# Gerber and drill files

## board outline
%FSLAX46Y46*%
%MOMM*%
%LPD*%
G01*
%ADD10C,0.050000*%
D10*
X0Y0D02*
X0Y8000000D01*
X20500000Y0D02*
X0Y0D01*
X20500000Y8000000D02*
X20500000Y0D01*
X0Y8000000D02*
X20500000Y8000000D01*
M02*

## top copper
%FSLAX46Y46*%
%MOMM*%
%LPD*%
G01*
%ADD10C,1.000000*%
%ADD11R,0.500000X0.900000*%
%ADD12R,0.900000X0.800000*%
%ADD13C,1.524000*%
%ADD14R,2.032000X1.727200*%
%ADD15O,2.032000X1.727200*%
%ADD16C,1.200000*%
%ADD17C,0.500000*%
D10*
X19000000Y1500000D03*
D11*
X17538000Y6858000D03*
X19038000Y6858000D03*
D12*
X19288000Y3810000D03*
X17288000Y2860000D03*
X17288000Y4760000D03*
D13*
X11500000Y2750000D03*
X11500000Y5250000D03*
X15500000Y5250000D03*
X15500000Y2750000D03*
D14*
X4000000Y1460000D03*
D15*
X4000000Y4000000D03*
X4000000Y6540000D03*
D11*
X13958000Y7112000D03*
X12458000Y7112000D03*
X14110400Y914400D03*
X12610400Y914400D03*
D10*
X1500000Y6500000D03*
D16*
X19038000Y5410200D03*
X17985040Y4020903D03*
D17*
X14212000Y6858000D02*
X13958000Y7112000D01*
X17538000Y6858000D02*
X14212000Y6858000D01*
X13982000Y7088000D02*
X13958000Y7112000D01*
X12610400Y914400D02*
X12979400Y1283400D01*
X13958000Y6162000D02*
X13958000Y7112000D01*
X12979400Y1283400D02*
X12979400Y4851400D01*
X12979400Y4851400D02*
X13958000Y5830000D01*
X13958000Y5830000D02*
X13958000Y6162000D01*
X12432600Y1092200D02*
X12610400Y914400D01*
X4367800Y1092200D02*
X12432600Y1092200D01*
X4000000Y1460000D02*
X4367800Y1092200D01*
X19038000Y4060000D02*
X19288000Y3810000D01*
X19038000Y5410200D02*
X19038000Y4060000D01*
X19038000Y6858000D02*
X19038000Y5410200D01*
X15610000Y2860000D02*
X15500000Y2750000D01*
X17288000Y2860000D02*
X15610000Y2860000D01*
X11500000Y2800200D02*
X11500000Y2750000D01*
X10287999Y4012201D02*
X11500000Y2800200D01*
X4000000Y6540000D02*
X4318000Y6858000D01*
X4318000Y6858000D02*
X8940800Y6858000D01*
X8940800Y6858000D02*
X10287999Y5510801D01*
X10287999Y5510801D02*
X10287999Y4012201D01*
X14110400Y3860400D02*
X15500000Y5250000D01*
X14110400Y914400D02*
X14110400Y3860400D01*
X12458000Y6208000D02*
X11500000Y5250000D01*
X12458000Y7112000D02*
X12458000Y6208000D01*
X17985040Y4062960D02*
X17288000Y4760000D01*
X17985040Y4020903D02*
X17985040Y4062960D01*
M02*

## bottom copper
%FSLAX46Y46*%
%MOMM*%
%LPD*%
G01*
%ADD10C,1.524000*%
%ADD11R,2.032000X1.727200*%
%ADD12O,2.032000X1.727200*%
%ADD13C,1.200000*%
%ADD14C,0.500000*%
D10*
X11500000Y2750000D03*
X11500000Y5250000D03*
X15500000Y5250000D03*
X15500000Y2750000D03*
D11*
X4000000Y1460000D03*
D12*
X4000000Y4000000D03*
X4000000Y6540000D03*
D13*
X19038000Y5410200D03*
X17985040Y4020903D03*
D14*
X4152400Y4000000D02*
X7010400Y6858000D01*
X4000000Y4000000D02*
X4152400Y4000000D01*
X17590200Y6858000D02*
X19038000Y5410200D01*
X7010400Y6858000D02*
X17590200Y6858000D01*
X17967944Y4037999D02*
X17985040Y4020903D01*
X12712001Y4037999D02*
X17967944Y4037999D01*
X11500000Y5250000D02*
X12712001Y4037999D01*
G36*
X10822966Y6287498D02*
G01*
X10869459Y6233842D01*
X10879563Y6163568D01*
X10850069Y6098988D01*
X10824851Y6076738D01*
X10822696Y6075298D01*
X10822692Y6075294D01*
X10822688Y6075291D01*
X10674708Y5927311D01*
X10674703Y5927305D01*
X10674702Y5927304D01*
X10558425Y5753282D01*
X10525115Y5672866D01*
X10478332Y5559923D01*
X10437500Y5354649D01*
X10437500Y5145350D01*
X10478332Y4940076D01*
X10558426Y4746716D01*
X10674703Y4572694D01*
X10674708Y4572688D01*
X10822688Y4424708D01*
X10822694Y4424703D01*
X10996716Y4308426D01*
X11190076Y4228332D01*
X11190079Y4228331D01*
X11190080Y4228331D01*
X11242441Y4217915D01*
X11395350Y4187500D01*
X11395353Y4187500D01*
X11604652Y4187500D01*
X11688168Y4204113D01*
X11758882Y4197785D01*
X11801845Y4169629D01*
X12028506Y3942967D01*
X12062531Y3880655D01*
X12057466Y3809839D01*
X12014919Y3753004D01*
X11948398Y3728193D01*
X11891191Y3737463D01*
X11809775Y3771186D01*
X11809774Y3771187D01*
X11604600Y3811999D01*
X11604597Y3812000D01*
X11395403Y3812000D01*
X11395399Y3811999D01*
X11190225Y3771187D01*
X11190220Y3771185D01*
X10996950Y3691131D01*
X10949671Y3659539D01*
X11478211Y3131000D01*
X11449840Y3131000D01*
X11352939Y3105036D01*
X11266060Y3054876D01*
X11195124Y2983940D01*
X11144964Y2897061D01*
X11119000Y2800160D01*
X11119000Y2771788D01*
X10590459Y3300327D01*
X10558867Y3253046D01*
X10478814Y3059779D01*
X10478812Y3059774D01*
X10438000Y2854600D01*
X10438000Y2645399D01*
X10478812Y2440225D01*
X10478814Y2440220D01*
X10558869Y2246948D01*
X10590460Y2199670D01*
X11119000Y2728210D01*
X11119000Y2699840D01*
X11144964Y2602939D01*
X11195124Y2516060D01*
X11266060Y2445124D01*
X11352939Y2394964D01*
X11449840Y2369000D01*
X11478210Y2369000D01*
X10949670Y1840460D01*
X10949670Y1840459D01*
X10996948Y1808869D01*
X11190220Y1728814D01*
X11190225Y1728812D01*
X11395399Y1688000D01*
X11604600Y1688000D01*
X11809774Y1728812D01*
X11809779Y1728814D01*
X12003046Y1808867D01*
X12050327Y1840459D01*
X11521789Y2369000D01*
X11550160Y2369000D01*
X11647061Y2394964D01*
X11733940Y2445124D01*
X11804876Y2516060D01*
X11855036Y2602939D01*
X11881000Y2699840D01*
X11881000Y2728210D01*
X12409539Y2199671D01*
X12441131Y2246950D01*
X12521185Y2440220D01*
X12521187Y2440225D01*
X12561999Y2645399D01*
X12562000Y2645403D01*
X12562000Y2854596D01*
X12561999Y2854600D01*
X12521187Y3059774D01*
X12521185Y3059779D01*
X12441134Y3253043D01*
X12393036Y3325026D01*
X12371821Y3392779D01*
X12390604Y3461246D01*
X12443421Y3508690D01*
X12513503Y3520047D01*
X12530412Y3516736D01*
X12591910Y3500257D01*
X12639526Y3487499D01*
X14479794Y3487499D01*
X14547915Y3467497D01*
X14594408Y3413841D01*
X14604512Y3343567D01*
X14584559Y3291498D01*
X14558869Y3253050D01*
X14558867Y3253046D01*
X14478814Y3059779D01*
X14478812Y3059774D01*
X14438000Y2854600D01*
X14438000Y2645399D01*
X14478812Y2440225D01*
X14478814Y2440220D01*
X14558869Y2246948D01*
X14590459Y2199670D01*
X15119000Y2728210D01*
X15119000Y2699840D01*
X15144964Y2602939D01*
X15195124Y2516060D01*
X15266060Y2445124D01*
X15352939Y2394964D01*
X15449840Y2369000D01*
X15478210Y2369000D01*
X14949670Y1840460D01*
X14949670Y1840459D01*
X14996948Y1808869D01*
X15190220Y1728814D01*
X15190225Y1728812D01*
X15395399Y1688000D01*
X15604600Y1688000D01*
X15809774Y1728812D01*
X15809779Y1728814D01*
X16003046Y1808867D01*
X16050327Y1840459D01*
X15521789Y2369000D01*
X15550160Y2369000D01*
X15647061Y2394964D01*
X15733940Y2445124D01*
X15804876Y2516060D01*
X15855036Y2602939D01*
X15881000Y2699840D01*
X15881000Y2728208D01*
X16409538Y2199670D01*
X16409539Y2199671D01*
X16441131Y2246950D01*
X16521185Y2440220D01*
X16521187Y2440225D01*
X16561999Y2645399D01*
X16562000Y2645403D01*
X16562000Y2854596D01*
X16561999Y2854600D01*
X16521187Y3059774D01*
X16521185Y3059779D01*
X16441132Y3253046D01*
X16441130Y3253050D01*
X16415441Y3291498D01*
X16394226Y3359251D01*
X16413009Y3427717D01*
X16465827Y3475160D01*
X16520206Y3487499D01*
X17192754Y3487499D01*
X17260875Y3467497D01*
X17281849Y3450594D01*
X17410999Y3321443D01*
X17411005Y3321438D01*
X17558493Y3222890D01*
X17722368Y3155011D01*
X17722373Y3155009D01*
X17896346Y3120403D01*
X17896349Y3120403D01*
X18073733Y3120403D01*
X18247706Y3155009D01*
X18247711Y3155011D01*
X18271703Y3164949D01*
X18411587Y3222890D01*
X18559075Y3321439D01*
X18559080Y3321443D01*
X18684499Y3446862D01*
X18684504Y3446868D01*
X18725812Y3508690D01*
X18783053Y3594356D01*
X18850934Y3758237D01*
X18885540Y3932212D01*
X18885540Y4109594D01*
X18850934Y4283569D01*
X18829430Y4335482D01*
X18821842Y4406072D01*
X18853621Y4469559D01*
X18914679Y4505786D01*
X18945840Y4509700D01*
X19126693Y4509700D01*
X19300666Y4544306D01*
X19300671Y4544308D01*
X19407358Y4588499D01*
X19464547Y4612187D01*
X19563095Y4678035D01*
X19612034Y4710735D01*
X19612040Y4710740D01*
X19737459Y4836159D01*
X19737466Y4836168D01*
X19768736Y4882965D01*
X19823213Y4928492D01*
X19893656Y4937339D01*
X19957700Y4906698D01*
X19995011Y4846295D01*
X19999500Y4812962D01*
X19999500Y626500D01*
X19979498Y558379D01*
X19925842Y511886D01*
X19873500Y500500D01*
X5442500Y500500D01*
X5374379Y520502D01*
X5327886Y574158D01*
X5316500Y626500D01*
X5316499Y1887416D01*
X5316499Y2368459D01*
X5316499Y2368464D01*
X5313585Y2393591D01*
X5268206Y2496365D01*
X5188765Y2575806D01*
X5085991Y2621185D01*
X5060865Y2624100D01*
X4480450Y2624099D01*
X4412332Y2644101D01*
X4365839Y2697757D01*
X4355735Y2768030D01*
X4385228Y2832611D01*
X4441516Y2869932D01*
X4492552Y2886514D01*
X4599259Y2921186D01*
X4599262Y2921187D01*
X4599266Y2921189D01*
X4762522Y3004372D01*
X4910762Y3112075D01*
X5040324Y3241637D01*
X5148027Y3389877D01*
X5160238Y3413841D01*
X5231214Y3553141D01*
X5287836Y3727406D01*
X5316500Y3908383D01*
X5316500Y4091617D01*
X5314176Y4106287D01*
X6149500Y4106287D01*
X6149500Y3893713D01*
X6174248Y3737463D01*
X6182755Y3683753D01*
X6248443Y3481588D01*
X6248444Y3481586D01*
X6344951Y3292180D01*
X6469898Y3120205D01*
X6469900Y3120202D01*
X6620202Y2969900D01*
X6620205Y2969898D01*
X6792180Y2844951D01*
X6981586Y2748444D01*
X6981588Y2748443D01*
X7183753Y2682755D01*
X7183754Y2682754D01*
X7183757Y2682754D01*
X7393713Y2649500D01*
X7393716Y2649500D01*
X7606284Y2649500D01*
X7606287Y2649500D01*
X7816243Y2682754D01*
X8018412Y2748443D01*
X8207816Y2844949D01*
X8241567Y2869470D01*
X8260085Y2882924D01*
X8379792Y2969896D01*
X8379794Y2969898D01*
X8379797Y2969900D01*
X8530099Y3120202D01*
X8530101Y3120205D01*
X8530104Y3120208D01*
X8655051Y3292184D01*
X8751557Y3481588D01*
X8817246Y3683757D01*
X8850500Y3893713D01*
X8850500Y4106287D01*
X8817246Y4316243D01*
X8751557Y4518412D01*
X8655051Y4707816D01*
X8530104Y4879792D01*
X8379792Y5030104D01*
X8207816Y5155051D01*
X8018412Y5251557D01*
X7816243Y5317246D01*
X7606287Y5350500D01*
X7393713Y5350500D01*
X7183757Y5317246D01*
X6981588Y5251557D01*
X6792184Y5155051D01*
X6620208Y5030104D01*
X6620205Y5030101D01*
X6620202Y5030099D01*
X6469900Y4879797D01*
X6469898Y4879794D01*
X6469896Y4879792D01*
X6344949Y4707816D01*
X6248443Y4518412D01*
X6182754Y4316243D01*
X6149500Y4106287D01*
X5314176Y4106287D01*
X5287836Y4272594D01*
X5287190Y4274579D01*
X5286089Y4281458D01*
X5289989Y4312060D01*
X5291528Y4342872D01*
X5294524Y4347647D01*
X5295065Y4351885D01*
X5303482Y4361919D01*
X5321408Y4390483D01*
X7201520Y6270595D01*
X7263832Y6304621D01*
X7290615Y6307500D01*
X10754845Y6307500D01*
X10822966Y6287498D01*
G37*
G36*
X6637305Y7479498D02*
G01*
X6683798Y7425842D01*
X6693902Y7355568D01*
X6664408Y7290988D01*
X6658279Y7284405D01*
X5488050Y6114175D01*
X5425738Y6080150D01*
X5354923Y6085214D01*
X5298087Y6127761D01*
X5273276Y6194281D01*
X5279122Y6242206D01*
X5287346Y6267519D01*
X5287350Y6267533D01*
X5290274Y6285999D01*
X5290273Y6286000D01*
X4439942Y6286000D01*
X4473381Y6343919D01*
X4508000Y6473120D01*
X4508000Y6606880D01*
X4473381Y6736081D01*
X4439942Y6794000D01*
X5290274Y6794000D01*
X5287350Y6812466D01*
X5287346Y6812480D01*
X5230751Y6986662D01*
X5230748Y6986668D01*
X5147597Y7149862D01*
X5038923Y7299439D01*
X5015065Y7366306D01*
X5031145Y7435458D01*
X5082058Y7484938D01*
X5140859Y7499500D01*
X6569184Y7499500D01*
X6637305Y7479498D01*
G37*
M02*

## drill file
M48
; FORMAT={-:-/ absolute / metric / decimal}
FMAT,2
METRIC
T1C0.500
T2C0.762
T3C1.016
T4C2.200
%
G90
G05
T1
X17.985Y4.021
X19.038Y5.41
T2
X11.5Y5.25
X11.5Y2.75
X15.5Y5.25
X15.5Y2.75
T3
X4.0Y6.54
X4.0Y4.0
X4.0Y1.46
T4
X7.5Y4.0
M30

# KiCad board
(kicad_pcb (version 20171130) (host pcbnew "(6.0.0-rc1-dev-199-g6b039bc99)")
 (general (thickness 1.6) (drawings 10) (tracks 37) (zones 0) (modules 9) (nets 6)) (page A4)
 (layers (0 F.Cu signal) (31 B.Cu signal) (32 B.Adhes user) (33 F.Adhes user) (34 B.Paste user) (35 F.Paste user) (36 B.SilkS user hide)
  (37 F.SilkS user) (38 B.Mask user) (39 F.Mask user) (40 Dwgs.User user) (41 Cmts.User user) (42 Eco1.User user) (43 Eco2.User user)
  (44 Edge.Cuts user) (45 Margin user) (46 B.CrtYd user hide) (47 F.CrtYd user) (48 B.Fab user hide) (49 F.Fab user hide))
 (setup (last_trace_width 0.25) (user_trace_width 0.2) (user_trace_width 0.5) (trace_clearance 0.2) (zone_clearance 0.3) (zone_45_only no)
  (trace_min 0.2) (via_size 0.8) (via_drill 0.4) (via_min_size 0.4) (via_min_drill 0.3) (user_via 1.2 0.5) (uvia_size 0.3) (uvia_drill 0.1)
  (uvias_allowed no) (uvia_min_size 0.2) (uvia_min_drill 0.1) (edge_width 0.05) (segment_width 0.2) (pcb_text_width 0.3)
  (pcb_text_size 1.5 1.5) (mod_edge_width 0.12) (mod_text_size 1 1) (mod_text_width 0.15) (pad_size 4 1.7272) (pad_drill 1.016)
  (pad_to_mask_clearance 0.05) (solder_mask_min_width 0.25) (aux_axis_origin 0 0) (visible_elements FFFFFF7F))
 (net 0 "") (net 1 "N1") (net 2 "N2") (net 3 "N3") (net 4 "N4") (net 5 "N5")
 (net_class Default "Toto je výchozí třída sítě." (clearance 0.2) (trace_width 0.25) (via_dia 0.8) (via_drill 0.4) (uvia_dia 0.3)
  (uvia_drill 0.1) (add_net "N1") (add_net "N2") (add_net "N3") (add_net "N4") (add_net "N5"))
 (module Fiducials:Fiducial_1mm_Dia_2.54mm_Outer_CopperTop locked (layer F.Cu) (at 19 -1.5)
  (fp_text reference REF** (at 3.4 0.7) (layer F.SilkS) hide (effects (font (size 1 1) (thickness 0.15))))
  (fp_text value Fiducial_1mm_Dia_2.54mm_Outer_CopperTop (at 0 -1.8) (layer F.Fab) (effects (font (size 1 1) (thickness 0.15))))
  (pad ~ smd circle (at 0 0) (size 1 1) (layers F.Cu F.Mask) (solder_mask_margin 0.77) (clearance 0.77)))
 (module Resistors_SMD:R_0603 (layer F.Cu) (at 18.288 -6.858 180)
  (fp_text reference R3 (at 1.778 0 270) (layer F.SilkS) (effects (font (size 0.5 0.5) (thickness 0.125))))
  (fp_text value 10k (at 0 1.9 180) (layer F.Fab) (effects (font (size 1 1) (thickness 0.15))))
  (pad 2 smd rect (at 0.75 0 180) (size 0.5 0.9) (layers F.Cu F.Paste F.Mask) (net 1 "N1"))
  (pad 1 smd rect (at -0.75 0 180) (size 0.5 0.9) (layers F.Cu F.Paste F.Mask) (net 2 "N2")))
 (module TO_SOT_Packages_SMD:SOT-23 (layer F.Cu) (at 18.288 -3.81)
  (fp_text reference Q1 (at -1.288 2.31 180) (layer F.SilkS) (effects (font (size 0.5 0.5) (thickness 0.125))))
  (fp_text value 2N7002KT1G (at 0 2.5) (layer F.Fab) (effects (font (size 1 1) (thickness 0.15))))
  (pad 3 smd rect (at 1 0) (size 0.9 0.8) (layers F.Cu F.Paste F.Mask) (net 2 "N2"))
  (pad 2 smd rect (at -1 0.95) (size 0.9 0.8) (layers F.Cu F.Paste F.Mask) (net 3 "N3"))
  (pad 1 smd rect (at -1 -0.95) (size 0.9 0.8) (layers F.Cu F.Paste F.Mask) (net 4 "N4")))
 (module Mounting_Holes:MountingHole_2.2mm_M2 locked (layer F.Cu) (at 7.5 -4)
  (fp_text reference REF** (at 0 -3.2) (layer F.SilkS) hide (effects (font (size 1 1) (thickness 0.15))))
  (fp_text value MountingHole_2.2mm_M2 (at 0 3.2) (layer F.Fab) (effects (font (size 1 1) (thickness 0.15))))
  (pad 1 np_thru_hole circle (at 0 0) (size 2.2 2.2) (drill 2.2) (layers *.Cu *.Mask)))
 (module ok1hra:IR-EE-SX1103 (layer F.Cu) (at 13.5 -4 180)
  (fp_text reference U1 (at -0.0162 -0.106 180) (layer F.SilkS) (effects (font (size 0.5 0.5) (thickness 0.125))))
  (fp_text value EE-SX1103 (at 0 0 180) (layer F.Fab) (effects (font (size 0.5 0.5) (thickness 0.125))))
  (pad 3 thru_hole circle (at 2 -1.25 180) (size 1.524 1.524) (drill 0.762) (layers *.Cu *.Mask) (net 3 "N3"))
  (pad 4 thru_hole circle (at 2 1.25 180) (size 1.524 1.524) (drill 0.762) (layers *.Cu *.Mask) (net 4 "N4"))
  (pad 1 thru_hole circle (at -2 1.25 180) (size 1.524 1.524) (drill 0.762) (layers *.Cu *.Mask) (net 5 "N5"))
  (pad 2 thru_hole circle (at -2 -1.25 180) (size 1.524 1.524) (drill 0.762) (layers *.Cu *.Mask) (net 3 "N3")))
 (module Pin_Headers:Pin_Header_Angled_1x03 (layer F.Cu) (at 4 -1.46 180)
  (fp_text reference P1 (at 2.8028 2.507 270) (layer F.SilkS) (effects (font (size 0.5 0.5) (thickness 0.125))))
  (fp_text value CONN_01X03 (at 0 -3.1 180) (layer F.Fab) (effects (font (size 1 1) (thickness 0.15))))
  (pad 1 thru_hole rect (at 0 0 180) (size 2.032 1.7272) (drill 1.016) (layers *.Cu *.Mask) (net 1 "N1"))
  (pad 2 thru_hole oval (at 0 2.54 180) (size 2.032 1.7272) (drill 1.016) (layers *.Cu *.Mask) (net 2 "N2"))
  (pad 3 thru_hole oval (at 0 5.08 180) (size 2.032 1.7272) (drill 1.016) (layers *.Cu *.Mask) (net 3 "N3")))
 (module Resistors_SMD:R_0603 (layer F.Cu) (at 13.208 -7.112 180)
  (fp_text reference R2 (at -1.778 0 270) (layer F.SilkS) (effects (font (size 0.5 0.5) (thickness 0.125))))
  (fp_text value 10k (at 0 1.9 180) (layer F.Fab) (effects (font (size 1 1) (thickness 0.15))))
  (pad 1 smd rect (at -0.75 0 180) (size 0.5 0.9) (layers F.Cu F.Paste F.Mask) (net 1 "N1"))
  (pad 2 smd rect (at 0.75 0 180) (size 0.5 0.9) (layers F.Cu F.Paste F.Mask) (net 4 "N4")))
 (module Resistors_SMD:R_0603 (layer F.Cu) (at 13.3604 -0.9144 180)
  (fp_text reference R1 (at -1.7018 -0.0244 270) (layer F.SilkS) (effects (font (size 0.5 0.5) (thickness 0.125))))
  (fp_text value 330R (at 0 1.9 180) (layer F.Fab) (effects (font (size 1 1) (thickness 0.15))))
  (pad 1 smd rect (at -0.75 0 180) (size 0.5 0.9) (layers F.Cu F.Paste F.Mask) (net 5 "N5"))
  (pad 2 smd rect (at 0.75 0 180) (size 0.5 0.9) (layers F.Cu F.Paste F.Mask) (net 1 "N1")))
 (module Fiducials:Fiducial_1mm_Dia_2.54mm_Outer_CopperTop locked (layer F.Cu) (at 1.5 -6.5)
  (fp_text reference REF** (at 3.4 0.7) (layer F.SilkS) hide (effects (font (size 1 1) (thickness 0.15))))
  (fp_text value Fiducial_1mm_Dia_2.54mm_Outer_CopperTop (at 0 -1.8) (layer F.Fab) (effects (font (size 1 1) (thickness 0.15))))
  (pad ~ smd circle (at 0 0) (size 1 1) (layers F.Cu F.Mask) (solder_mask_margin 0.77) (clearance 0.77)))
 (gr_line (start 0 0) (end 0 -8) (layer Edge.Cuts) (width 0.05))
 (gr_line (start 20.5 0) (end 0 0) (layer Edge.Cuts) (width 0.05))
 (gr_line (start 20.5 -8) (end 20.5 0) (layer Edge.Cuts) (width 0.05))
 (gr_line (start 0 -8) (end 20.5 -8) (layer Edge.Cuts) (width 0.05))
 (segment (start 14.212 -6.858) (end 13.958 -7.112) (width 0.5) (layer F.Cu) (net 1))
 (segment (start 17.538 -6.858) (end 14.212 -6.858) (width 0.5) (layer F.Cu) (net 1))
 (segment (start 13.982 -7.088) (end 13.958 -7.112) (width 0.5) (layer F.Cu) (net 1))
 (segment (start 12.6104 -0.9144) (end 12.9794 -1.2834) (width 0.5) (layer F.Cu) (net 1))
 (segment (start 13.958 -6.162) (end 13.958 -7.112) (width 0.5) (layer F.Cu) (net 1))
 (segment (start 12.9794 -1.2834) (end 12.9794 -4.8514) (width 0.5) (layer F.Cu) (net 1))
 (segment (start 12.9794 -4.8514) (end 13.958 -5.83) (width 0.5) (layer F.Cu) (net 1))
 (segment (start 13.958 -5.83) (end 13.958 -6.162) (width 0.5) (layer F.Cu) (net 1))
 (segment (start 12.4326 -1.0922) (end 12.6104 -0.9144) (width 0.5) (layer F.Cu) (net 1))
 (segment (start 4.3678 -1.0922) (end 12.4326 -1.0922) (width 0.5) (layer F.Cu) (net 1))
 (segment (start 4 -1.46) (end 4.3678 -1.0922) (width 0.5) (layer F.Cu) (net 1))
 (segment (start 19.038 -4.06) (end 19.288 -3.81) (width 0.5) (layer F.Cu) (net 2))
 (segment (start 4.1524 -4) (end 7.0104 -6.858) (width 0.5) (layer B.Cu) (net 2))
 (segment (start 4 -4) (end 4.1524 -4) (width 0.5) (layer B.Cu) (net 2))
 (segment (start 19.038 -5.4102) (end 19.038 -4.06) (width 0.5) (layer F.Cu) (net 2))
 (segment (start 19.038 -6.858) (end 19.038 -5.4102) (width 0.5) (layer F.Cu) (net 2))
 (segment (start 17.5902 -6.858) (end 19.038 -5.4102) (width 0.5) (layer B.Cu) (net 2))
 (via (at 19.038 -5.4102) (size 1.2) (drill 0.5) (layers F.Cu B.Cu) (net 2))
 (segment (start 7.0104 -6.858) (end 17.5902 -6.858) (width 0.5) (layer B.Cu) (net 2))
 (segment (start 15.61 -2.86) (end 15.5 -2.75) (width 0.5) (layer F.Cu) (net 3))
 (segment (start 17.288 -2.86) (end 15.61 -2.86) (width 0.5) (layer F.Cu) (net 3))
 (segment (start 11.5 -2.8002) (end 11.5 -2.75) (width 0.5) (layer F.Cu) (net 3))
 (segment (start 10.287999 -4.012201) (end 11.5 -2.8002) (width 0.5) (layer F.Cu) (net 3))
 (segment (start 4 -6.54) (end 4.318 -6.858) (width 0.5) (layer F.Cu) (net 3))
 (segment (start 4.318 -6.858) (end 8.9408 -6.858) (width 0.5) (layer F.Cu) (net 3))
 (segment (start 8.9408 -6.858) (end 10.287999 -5.510801) (width 0.5) (layer F.Cu) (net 3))
 (segment (start 10.287999 -5.510801) (end 10.287999 -4.012201) (width 0.5) (layer F.Cu) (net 3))
 (segment (start 14.1104 -3.8604) (end 15.5 -5.25) (width 0.5) (layer F.Cu) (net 5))
 (segment (start 14.1104 -0.9144) (end 14.1104 -3.8604) (width 0.5) (layer F.Cu) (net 5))
 (segment (start 12.458 -6.208) (end 11.5 -5.25) (width 0.5) (layer F.Cu) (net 4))
 (segment (start 12.458 -7.112) (end 12.458 -6.208) (width 0.5) (layer F.Cu) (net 4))
 (segment (start 17.967944 -4.037999) (end 17.98504 -4.020903) (width 0.5) (layer B.Cu) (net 4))
 (segment (start 12.712001 -4.037999) (end 17.967944 -4.037999) (width 0.5) (layer B.Cu) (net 4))
 (via (at 17.98504 -4.020903) (size 1.2) (drill 0.5) (layers F.Cu B.Cu) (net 4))
 (segment (start 11.5 -5.25) (end 12.712001 -4.037999) (width 0.5) (layer B.Cu) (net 4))
 (segment (start 17.98504 -4.06296) (end 17.288 -4.76) (width 0.5) (layer F.Cu) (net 4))
 (segment (start 17.98504 -4.020903) (end 17.98504 -4.06296) (width 0.5) (layer F.Cu) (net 4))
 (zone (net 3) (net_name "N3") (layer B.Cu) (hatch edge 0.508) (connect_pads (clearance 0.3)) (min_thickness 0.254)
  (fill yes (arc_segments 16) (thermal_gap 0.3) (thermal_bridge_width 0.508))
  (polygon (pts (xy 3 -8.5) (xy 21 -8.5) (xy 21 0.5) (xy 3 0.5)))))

